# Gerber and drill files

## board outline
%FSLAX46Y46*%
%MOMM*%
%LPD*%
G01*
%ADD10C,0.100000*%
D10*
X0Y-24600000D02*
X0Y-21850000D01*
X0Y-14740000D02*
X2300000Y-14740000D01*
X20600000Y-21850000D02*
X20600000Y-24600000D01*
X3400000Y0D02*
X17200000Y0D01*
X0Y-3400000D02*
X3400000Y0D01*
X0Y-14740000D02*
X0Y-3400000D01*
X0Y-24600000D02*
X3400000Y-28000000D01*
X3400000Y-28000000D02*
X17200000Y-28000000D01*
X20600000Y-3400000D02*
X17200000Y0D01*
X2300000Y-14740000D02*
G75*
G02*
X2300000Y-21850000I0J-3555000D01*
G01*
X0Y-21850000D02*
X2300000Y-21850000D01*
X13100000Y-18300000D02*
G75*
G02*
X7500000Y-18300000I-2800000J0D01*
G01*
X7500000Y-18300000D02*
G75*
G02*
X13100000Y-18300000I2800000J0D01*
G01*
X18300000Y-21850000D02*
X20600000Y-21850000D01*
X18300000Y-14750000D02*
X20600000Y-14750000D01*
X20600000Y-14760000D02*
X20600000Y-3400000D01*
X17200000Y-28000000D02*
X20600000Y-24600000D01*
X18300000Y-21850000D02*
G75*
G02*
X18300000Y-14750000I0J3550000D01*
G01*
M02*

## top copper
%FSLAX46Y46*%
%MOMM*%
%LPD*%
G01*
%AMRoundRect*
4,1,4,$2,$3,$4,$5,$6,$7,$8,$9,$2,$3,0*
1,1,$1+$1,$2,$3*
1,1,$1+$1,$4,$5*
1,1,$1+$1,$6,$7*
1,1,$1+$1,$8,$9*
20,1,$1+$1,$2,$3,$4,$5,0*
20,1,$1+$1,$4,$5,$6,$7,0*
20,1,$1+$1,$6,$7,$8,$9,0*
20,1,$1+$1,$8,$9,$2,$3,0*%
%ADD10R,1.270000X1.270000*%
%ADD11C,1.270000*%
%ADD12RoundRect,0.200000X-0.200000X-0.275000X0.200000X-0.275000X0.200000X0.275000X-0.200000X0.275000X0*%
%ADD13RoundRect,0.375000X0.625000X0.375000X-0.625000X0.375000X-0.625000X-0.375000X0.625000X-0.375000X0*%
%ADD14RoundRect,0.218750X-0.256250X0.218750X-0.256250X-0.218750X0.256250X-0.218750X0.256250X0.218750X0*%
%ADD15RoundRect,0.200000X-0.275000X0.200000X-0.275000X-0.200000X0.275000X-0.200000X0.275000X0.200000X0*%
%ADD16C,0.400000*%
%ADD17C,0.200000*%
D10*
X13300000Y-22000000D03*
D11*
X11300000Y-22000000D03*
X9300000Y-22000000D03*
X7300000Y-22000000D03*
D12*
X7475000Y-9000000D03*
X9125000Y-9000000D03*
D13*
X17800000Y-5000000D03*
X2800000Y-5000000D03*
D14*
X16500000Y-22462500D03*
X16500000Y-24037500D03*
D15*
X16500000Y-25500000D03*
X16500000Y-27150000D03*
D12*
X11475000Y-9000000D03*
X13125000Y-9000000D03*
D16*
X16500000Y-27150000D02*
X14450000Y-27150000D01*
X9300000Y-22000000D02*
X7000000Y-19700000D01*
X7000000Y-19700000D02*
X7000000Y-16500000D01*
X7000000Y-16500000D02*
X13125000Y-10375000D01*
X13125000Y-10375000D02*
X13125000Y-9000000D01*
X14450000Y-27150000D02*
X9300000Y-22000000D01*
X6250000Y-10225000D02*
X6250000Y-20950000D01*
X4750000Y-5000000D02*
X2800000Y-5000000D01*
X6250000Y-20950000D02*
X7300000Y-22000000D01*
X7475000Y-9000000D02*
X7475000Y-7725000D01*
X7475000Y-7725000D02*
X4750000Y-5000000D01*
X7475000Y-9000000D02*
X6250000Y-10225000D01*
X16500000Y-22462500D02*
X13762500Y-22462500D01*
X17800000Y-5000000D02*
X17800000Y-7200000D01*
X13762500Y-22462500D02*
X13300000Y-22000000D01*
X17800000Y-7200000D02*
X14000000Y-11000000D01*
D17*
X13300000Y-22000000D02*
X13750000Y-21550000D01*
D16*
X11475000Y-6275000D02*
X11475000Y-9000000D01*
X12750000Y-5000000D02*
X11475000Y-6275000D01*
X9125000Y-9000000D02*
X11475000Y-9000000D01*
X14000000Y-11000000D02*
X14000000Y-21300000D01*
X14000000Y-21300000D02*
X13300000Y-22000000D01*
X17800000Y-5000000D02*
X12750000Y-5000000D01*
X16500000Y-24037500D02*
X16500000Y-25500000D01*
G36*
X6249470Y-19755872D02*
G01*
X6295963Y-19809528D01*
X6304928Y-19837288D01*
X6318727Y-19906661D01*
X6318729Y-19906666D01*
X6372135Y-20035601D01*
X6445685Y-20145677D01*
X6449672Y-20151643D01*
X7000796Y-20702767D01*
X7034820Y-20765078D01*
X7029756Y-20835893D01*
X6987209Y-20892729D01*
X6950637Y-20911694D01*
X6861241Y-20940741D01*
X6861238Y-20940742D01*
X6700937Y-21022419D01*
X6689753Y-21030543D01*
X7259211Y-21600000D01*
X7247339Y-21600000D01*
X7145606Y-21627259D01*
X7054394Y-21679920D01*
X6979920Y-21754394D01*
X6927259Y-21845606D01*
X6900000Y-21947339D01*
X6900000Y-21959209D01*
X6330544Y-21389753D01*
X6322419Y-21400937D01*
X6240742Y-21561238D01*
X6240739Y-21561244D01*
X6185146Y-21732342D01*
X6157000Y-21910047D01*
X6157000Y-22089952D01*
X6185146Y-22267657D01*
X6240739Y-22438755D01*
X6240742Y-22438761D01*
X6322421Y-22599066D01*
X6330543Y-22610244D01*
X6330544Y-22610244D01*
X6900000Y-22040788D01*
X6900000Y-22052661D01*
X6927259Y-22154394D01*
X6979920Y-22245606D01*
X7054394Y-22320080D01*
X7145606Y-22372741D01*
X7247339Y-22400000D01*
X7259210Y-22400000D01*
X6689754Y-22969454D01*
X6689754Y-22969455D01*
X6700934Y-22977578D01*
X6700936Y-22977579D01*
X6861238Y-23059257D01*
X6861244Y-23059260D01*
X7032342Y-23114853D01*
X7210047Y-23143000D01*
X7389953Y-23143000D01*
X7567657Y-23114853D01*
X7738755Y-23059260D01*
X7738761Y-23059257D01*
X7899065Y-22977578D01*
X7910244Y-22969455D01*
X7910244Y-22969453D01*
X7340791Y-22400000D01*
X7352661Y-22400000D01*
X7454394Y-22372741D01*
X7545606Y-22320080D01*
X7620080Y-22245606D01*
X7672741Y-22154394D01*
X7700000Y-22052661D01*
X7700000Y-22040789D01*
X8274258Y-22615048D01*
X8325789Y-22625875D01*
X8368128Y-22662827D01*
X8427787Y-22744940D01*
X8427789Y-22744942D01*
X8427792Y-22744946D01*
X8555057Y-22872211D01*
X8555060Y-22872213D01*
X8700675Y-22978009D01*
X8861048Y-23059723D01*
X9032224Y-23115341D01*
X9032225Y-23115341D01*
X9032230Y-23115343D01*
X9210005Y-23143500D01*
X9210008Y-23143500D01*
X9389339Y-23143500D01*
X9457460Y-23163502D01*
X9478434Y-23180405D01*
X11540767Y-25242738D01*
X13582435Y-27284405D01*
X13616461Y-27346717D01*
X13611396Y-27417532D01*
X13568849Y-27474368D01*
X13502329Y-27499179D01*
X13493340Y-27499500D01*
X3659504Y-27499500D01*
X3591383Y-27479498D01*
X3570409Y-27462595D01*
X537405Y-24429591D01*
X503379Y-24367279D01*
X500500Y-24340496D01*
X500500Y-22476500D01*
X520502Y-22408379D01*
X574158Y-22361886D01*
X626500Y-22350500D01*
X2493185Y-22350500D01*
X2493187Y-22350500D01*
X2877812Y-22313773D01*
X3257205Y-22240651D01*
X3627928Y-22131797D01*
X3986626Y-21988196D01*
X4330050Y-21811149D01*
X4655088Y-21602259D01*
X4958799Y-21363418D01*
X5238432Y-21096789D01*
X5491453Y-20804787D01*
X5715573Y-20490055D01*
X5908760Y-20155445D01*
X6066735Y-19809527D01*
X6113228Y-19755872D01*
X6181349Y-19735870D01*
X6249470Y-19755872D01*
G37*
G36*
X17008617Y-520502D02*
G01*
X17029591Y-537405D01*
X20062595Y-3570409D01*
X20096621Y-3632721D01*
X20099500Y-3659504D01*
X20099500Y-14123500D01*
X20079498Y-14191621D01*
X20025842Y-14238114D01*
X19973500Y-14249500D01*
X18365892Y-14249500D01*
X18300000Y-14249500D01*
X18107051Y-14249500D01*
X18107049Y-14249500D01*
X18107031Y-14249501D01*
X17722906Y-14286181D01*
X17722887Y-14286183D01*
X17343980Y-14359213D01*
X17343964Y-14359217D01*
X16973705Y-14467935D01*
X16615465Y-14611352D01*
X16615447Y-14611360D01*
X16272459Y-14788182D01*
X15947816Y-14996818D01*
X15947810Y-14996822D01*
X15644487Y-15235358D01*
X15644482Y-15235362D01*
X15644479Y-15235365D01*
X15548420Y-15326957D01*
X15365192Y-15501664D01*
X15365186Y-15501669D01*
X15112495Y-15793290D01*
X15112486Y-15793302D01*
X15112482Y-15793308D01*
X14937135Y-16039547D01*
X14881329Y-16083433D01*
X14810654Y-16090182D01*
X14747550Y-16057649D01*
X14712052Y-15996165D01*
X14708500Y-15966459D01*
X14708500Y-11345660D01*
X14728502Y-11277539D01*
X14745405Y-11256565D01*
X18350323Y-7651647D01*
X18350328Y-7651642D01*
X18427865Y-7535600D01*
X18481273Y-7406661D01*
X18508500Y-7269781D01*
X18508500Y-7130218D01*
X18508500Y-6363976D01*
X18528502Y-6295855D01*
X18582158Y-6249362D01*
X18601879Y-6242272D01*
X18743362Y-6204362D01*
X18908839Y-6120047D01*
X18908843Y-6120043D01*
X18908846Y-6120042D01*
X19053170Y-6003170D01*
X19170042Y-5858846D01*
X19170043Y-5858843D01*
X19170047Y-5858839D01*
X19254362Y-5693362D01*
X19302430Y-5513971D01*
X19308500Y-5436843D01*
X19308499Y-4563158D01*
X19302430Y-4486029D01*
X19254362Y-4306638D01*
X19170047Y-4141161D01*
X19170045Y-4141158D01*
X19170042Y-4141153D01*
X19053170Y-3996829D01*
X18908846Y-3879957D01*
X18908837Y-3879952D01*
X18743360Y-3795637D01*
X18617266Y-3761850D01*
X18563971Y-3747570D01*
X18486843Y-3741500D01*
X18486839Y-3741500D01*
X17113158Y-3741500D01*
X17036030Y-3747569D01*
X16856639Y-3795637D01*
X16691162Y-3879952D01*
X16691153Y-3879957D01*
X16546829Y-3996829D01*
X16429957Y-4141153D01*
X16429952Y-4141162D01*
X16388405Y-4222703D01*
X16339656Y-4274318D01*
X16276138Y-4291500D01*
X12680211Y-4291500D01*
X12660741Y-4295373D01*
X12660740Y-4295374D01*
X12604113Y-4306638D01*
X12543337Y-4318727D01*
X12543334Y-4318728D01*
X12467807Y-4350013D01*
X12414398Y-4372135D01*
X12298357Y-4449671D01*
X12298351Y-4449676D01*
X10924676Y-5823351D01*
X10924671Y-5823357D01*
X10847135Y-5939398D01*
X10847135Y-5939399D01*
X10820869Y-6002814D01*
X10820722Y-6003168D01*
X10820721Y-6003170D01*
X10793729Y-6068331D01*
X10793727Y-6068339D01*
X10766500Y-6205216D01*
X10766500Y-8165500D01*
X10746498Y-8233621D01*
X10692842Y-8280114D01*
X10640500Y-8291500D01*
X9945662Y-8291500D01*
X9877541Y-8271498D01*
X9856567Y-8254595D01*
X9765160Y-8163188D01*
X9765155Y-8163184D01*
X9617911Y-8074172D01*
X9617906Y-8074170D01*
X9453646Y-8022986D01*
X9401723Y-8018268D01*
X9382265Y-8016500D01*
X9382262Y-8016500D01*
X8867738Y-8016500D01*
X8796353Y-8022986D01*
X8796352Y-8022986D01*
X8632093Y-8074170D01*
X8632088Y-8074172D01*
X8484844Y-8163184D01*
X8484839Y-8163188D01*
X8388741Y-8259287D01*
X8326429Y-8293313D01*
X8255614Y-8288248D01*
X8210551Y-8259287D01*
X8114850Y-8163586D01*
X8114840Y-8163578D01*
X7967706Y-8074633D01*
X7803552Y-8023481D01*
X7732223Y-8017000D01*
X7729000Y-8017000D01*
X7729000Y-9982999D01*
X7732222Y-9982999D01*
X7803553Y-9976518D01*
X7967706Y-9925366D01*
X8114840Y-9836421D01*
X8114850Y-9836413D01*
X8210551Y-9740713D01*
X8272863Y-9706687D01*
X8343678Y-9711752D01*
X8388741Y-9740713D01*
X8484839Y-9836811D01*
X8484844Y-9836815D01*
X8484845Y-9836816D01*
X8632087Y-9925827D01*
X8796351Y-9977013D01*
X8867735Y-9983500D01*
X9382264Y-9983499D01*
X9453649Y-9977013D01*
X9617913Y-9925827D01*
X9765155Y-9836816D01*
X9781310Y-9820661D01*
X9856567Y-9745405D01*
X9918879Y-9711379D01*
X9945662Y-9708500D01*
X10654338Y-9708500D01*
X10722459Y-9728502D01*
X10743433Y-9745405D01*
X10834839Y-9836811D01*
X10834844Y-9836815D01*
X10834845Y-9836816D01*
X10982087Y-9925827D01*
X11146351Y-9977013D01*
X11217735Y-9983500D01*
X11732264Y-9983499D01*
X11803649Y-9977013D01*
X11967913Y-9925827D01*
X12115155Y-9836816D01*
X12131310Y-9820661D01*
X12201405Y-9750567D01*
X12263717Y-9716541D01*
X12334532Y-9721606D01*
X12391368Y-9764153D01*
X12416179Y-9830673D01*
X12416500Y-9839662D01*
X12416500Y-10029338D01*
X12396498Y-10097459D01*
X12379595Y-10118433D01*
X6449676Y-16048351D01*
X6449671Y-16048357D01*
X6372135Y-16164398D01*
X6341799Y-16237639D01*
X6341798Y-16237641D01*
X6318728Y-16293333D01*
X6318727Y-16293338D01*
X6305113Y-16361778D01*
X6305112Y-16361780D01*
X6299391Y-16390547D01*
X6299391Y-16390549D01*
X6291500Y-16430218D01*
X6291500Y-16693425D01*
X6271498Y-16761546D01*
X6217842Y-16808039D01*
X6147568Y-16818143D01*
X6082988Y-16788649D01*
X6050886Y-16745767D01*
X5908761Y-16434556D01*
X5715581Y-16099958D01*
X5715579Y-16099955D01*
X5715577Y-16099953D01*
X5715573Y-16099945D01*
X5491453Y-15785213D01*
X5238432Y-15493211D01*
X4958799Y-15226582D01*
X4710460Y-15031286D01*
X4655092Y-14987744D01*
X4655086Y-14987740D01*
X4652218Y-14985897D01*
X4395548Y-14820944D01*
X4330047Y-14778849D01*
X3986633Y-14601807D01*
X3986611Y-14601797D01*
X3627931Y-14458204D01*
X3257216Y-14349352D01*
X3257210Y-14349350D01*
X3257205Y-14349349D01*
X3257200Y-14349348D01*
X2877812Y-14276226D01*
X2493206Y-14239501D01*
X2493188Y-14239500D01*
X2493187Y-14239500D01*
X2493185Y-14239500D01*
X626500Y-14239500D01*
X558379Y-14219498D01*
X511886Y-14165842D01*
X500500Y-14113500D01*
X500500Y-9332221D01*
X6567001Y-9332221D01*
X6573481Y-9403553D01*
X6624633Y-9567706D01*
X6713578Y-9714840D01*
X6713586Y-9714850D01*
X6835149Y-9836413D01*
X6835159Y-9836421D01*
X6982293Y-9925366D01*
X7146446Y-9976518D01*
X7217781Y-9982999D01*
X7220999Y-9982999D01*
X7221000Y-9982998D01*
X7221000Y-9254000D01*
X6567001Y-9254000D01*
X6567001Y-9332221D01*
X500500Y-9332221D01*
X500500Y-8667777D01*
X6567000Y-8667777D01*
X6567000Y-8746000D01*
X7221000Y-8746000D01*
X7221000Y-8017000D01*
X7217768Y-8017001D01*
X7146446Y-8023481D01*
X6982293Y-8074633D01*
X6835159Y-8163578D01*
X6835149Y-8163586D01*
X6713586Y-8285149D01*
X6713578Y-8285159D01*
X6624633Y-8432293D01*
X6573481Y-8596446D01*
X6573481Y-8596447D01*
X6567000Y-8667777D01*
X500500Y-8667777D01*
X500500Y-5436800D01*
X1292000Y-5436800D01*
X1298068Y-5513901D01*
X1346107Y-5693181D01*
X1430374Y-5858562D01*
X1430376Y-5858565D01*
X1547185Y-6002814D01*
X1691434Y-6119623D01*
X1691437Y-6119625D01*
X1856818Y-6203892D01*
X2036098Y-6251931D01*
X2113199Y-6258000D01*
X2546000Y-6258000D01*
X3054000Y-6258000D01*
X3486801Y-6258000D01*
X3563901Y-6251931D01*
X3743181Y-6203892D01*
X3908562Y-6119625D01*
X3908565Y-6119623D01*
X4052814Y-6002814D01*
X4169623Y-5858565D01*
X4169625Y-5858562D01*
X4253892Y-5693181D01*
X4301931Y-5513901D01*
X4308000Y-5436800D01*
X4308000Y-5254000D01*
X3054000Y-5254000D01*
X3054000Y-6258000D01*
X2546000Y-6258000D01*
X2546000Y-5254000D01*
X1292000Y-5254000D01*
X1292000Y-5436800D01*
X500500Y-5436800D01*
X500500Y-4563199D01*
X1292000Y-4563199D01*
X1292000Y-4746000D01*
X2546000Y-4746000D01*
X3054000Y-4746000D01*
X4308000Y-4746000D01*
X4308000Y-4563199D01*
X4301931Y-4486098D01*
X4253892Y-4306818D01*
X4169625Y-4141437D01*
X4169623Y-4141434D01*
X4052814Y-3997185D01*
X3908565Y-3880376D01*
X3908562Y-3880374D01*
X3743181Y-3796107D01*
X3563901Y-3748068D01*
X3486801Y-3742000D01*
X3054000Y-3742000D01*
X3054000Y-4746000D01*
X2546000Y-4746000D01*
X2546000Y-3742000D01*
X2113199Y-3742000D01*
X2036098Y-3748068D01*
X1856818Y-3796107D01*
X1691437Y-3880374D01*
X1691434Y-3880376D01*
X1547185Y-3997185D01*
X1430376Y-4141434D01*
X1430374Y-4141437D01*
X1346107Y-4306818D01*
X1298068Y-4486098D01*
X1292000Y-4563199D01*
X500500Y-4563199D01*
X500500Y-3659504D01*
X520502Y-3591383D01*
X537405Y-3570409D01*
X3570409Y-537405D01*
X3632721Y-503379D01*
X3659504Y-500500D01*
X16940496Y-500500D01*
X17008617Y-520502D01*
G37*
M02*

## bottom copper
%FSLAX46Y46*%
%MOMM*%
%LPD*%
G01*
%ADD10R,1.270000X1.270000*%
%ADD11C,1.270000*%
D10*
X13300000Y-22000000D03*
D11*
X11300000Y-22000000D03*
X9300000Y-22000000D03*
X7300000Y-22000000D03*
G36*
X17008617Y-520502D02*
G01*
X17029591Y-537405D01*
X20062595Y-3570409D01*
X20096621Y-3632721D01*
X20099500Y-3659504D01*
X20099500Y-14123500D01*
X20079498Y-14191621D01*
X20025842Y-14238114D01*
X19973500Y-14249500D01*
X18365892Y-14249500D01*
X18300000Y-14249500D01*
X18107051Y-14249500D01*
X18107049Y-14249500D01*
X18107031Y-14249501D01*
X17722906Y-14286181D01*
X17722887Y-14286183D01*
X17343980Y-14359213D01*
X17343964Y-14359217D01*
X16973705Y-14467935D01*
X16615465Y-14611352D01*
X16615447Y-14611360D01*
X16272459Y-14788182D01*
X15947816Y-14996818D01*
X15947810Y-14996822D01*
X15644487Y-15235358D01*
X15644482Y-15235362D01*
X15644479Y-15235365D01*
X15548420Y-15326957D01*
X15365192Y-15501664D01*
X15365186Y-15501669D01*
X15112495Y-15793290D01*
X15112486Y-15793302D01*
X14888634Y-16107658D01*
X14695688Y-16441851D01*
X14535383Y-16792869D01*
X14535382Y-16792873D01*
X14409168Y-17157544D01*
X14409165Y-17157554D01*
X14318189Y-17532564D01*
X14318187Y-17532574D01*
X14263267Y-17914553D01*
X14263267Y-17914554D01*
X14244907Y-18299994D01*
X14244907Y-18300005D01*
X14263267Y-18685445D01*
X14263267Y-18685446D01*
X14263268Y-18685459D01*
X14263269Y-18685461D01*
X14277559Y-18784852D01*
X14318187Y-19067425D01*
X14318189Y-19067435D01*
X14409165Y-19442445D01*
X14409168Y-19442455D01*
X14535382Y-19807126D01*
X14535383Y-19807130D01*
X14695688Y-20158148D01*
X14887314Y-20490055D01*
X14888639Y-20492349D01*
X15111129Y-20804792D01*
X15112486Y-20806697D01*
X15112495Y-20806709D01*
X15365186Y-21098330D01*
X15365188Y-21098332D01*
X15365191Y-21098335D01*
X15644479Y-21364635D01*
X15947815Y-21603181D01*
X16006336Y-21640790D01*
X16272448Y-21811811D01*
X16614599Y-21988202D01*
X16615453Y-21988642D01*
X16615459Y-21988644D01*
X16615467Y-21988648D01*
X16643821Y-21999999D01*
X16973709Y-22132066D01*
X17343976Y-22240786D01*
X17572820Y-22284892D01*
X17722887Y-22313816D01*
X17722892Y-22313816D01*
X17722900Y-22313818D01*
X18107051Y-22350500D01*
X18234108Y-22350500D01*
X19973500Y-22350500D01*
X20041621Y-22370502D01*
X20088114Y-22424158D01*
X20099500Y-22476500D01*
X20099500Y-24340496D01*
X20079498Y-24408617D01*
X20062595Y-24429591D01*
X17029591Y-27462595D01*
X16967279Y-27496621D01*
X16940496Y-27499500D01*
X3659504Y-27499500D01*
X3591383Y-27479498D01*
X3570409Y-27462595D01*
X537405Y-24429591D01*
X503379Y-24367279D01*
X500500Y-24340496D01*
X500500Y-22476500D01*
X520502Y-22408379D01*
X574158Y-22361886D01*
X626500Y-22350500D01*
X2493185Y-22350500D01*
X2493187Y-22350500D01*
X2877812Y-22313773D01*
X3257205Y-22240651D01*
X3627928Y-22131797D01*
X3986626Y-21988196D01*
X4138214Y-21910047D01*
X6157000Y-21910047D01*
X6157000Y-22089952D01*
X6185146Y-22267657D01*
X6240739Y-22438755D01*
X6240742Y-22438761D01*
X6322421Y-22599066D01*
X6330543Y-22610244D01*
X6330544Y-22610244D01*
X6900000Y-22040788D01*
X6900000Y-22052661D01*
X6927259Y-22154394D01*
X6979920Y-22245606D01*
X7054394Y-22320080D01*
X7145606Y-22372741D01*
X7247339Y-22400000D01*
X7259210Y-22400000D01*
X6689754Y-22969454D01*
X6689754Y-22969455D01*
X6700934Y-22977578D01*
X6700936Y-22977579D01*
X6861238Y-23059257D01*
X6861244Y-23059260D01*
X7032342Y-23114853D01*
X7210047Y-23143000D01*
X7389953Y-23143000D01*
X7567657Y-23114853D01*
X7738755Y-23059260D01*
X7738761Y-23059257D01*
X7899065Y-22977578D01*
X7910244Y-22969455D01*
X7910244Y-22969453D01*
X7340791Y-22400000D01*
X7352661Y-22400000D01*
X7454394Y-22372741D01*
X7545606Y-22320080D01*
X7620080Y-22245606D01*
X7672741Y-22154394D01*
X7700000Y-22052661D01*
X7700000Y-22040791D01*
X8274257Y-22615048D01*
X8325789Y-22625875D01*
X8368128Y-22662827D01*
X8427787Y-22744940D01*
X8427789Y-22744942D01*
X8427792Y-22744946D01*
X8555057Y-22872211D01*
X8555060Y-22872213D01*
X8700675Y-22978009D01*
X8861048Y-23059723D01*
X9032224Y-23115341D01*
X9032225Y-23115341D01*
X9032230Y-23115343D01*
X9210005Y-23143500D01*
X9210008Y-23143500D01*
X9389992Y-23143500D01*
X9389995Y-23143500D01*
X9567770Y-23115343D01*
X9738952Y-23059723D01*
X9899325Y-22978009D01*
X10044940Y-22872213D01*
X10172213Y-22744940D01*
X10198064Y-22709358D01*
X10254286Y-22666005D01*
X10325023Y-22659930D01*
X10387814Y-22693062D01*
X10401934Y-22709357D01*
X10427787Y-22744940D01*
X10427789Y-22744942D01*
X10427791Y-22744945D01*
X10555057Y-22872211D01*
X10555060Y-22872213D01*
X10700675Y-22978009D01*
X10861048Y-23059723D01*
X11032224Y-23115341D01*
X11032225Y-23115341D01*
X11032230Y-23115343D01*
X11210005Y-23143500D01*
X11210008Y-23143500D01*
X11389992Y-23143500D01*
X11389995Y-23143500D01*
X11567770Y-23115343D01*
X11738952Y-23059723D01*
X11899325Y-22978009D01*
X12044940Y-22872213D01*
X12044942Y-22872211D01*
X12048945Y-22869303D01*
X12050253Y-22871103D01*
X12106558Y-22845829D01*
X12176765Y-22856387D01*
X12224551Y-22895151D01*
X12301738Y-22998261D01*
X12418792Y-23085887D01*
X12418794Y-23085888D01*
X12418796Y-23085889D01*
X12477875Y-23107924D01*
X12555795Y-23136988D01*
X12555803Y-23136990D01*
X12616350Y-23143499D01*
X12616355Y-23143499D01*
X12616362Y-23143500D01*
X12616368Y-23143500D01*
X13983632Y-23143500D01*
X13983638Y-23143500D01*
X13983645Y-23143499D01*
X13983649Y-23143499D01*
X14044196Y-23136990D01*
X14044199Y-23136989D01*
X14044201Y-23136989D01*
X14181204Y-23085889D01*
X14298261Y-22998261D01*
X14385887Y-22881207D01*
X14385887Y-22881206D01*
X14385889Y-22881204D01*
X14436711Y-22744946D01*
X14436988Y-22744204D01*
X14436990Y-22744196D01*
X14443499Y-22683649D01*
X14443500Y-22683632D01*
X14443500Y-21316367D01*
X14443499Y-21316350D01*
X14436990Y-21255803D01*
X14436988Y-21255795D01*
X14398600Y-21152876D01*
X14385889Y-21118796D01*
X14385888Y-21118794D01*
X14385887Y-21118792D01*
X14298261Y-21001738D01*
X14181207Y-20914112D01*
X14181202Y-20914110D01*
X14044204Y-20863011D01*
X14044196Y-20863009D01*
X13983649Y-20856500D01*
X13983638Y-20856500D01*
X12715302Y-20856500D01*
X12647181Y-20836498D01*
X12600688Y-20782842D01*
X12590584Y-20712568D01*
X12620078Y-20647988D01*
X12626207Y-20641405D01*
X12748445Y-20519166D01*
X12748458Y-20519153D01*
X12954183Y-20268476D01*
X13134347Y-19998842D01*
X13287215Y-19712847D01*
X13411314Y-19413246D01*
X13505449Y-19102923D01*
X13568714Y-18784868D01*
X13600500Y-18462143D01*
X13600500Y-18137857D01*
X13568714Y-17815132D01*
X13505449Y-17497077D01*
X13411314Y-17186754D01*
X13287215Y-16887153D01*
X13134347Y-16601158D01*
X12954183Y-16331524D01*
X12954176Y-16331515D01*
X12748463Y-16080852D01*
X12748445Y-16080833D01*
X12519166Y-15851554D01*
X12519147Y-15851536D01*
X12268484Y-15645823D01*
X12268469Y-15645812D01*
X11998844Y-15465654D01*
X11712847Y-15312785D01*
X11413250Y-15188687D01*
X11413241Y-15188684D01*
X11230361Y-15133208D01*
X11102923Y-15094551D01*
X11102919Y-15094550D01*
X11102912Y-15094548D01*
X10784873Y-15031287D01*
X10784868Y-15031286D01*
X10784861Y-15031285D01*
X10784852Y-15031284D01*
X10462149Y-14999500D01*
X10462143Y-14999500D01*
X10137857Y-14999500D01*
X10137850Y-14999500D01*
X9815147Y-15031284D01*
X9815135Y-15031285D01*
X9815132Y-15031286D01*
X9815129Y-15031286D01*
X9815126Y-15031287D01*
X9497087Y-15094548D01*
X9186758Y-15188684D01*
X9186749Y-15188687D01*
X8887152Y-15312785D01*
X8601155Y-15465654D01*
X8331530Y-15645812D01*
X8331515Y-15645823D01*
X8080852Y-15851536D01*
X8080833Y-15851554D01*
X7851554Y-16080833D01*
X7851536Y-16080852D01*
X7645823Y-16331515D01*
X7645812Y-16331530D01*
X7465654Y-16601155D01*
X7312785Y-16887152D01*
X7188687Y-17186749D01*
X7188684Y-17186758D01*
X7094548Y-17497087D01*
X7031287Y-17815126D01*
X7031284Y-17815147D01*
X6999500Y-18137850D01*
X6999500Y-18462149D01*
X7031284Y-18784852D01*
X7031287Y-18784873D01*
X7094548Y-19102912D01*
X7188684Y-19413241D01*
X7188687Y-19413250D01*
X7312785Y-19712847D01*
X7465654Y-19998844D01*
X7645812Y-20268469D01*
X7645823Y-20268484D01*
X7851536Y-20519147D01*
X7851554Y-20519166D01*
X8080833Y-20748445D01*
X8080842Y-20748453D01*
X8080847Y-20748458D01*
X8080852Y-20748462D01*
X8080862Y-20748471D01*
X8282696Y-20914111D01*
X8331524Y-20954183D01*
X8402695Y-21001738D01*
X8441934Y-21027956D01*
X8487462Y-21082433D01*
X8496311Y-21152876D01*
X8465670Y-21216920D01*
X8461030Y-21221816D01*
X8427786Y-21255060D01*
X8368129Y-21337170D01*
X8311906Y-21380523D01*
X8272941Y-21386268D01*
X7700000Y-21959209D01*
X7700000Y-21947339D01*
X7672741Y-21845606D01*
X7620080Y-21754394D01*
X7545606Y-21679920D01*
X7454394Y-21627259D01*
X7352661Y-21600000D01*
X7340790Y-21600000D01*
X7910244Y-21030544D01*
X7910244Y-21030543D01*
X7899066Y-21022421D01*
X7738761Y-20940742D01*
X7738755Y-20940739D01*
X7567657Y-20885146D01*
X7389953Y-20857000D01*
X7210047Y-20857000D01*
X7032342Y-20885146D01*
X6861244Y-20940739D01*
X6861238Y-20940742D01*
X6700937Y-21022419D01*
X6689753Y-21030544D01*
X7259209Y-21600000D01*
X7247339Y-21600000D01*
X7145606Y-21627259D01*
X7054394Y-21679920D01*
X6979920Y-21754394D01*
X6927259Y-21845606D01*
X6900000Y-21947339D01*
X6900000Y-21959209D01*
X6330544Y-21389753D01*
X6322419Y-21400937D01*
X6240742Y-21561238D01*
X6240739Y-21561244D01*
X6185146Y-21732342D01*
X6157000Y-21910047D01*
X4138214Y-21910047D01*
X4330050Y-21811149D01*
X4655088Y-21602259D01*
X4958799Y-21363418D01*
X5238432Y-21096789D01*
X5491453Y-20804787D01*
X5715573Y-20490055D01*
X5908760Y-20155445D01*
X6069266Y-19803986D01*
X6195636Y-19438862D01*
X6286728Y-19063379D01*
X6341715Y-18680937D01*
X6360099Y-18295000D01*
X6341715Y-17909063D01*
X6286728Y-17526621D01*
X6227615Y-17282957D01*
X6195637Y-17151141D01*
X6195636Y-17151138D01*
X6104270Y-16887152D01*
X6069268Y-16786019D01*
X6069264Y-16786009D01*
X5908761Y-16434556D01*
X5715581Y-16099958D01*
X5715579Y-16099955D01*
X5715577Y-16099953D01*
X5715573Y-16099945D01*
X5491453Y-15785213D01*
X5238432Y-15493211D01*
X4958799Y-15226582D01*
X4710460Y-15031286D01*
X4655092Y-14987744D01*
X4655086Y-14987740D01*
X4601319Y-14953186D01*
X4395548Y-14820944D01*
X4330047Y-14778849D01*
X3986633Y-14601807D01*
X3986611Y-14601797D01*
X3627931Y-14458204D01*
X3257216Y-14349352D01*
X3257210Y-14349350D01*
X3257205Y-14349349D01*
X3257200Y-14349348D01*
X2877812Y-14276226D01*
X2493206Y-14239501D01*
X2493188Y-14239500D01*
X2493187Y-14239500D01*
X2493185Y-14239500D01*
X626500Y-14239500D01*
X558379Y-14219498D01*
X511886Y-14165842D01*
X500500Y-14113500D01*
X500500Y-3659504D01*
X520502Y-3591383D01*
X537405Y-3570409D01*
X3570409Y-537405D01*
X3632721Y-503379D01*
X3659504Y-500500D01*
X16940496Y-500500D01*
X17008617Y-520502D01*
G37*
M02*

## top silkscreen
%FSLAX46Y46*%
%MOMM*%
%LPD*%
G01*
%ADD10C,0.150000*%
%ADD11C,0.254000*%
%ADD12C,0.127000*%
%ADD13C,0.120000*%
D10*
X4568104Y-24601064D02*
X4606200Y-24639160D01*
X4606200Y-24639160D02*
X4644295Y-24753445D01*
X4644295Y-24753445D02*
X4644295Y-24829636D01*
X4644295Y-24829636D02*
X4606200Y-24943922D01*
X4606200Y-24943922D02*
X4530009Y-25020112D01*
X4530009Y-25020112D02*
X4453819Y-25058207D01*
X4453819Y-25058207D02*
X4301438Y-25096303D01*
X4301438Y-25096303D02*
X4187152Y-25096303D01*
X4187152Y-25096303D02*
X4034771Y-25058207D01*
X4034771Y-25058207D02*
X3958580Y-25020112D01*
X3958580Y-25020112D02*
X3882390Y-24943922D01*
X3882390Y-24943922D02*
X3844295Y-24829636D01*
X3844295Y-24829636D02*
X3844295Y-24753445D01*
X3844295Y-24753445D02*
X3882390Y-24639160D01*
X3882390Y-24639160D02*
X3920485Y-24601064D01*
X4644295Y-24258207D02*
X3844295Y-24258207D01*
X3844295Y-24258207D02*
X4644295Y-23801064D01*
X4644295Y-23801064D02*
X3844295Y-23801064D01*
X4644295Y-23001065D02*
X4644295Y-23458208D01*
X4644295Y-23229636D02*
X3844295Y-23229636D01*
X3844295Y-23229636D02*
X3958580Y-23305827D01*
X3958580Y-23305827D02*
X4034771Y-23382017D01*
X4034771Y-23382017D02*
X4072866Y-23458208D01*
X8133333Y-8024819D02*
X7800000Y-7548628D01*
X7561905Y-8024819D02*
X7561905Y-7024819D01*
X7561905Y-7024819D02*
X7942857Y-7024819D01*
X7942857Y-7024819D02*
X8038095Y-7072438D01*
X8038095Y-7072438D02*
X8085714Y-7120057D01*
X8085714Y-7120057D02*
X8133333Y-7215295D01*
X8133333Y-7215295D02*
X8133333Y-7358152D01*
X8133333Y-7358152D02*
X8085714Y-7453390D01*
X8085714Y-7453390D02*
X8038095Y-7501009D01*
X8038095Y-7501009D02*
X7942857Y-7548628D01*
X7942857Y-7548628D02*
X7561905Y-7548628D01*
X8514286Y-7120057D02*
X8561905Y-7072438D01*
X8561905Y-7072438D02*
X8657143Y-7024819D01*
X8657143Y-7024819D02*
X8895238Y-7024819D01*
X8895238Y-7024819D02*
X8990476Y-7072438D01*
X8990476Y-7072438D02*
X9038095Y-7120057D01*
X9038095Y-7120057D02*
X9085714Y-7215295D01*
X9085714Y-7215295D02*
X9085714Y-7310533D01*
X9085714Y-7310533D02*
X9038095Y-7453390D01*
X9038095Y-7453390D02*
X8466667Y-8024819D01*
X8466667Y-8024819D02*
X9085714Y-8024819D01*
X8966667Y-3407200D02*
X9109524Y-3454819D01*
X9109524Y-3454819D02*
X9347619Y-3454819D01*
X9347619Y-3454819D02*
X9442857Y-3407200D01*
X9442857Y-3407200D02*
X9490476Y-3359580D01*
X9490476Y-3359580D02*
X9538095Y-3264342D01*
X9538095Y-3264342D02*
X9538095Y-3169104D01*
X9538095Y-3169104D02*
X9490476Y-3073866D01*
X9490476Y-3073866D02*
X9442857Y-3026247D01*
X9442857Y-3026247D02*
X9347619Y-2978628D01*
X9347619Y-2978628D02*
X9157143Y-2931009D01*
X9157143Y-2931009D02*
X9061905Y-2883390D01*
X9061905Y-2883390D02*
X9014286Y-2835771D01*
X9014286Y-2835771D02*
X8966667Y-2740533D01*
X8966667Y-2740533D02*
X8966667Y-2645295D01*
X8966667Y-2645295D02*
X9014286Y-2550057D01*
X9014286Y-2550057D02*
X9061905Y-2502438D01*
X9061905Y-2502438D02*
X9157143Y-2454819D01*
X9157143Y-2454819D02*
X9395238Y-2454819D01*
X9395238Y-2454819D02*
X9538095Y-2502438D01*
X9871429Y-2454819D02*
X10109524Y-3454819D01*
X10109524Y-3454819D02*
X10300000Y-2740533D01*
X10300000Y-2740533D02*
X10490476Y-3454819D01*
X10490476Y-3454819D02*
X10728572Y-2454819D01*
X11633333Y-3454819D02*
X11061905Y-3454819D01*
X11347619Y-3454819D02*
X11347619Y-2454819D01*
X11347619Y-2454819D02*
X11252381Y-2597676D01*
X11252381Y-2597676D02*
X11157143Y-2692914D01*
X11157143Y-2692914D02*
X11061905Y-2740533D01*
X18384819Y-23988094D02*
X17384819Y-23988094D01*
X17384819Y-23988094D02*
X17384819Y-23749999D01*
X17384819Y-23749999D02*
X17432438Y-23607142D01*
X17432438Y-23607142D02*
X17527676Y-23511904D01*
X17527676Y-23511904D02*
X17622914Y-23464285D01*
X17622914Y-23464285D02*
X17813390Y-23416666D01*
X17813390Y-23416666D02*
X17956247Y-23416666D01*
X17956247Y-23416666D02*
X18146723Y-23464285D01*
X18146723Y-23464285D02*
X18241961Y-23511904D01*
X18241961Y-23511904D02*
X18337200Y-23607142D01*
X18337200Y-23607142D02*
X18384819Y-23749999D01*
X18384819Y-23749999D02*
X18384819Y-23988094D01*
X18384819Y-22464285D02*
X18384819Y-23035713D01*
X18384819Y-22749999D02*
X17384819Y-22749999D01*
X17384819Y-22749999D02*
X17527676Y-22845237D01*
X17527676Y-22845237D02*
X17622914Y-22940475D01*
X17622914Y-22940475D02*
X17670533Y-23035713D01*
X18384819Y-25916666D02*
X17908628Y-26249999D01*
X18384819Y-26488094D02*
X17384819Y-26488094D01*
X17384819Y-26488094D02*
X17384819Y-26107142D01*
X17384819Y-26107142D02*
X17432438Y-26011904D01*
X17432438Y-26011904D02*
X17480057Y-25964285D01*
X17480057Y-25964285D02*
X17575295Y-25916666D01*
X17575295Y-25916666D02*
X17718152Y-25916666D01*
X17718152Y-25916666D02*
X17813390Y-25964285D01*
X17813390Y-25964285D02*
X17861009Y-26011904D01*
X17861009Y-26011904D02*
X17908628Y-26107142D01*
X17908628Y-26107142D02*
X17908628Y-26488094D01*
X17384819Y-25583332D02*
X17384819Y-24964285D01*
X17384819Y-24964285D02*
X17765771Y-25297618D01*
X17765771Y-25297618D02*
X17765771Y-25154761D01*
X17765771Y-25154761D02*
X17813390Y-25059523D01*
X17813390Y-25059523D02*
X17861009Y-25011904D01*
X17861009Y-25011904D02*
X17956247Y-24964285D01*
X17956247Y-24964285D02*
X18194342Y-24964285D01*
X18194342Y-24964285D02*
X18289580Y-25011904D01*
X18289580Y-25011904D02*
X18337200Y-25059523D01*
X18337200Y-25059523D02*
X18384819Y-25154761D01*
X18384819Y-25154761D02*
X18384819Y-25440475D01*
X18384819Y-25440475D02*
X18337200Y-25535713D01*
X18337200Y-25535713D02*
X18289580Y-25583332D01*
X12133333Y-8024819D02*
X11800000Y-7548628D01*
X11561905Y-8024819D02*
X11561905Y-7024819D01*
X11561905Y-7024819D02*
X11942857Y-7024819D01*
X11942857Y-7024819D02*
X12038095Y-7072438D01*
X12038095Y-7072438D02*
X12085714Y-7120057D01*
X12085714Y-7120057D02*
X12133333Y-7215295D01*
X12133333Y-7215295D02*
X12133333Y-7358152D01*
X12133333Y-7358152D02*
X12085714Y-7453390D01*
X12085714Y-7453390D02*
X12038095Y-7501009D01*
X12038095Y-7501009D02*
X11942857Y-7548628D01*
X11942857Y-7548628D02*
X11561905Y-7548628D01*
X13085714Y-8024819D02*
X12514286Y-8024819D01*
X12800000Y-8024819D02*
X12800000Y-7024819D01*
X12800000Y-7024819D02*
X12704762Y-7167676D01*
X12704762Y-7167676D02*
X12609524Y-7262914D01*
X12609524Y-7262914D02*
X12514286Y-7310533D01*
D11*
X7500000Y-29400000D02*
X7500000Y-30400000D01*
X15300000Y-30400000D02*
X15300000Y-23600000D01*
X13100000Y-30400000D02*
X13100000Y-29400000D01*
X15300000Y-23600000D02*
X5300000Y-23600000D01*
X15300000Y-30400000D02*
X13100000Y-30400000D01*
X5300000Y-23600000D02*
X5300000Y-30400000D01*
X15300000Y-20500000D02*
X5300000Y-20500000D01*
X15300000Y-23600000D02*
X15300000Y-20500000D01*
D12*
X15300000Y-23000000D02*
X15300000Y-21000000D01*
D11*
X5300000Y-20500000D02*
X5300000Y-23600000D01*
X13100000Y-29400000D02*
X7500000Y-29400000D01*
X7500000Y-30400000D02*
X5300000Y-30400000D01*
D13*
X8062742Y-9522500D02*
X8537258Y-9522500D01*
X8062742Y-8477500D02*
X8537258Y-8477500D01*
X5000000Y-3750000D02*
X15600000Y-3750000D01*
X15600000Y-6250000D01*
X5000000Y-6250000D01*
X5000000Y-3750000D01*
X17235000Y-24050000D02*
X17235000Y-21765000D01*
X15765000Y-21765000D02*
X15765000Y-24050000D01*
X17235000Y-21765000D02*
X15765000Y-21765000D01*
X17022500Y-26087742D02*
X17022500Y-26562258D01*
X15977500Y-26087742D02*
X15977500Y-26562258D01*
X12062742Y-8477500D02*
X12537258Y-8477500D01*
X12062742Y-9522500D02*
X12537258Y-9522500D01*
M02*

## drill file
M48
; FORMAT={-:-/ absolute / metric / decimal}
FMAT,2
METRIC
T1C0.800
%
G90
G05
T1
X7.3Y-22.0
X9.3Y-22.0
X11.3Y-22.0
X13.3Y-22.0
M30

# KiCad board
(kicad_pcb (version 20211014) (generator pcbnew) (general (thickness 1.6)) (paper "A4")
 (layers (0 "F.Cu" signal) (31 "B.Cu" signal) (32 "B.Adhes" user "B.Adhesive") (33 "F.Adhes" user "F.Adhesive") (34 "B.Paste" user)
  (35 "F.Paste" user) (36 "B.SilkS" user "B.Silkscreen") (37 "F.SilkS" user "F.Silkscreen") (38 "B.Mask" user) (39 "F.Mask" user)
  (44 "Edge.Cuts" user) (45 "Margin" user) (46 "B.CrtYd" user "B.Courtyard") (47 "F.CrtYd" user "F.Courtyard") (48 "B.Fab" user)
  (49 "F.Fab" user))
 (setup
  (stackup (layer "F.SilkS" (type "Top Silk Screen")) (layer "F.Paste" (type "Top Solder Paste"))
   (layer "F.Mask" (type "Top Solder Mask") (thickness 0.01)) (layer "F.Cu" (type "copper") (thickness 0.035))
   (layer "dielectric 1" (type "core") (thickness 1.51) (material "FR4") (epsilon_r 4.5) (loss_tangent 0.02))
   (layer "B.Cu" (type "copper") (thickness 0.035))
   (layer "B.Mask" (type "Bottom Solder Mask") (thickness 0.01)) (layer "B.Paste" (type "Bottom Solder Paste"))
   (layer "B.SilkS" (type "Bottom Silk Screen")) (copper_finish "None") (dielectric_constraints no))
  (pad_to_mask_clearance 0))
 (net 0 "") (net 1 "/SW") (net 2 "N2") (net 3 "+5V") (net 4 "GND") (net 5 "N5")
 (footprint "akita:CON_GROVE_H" (layer "F.Cu") (at 10.3 22 180)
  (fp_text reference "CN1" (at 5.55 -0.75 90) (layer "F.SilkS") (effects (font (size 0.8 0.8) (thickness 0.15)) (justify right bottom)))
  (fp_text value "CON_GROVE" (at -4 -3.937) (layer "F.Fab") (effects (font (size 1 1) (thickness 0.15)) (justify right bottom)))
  (fp_line (start 2.8 -7.4) (end 2.8 -8.4) (layer "F.SilkS") (width 0.254))
  (fp_line (start -5 -8.4) (end -5 -1.6) (layer "F.SilkS") (width 0.254))
  (fp_line (start -2.8 -8.4) (end -2.8 -7.4) (layer "F.SilkS") (width 0.254))
  (fp_line (start -5 -1.6) (end 5 -1.6) (layer "F.SilkS") (width 0.254))
  (fp_line (start -5 -8.4) (end -2.8 -8.4) (layer "F.SilkS") (width 0.254))
  (fp_line (start 5 -1.6) (end 5 -8.4) (layer "F.SilkS") (width 0.254))
  (fp_line (start -5 1.5) (end 5 1.5) (layer "F.SilkS") (width 0.254))
  (fp_line (start -5 -1.6) (end -5 1.5) (layer "F.SilkS") (width 0.254))
  (fp_line (start -5 -1) (end -5 1) (layer "F.SilkS") (width 0.127))
  (fp_line (start 5 1.5) (end 5 -1.6) (layer "F.SilkS") (width 0.254))
  (fp_line (start -2.8 -7.4) (end 2.8 -7.4) (layer "F.SilkS") (width 0.254))
  (fp_line (start 2.8 -8.4) (end 5 -8.4) (layer "F.SilkS") (width 0.254))
  (pad "1" thru_hole rect locked (at -3 0 180) (size 1.27 1.27) (drill 0.8) (layers *.Cu *.Mask) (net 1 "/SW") (solder_mask_margin 0.1016))
  (pad "2" thru_hole circle locked (at -1 0 180) (size 1.27 1.27) (drill 0.8) (layers *.Cu *.Mask) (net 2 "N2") (solder_mask_margin 0.1016))
  (pad "3" thru_hole circle locked (at 1 0 180) (size 1.27 1.27) (drill 0.8) (layers *.Cu *.Mask) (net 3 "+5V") (solder_mask_margin 0.1016))
  (pad "4" thru_hole circle locked (at 3 0 180) (size 1.27 1.27) (drill 0.8) (layers *.Cu *.Mask) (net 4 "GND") (solder_mask_margin 0.1016)))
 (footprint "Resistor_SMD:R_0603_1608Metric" (layer "F.Cu") (at 8.3 9)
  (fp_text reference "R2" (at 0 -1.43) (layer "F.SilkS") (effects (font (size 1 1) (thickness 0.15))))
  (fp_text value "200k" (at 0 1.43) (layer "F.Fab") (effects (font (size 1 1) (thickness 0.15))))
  (fp_line (start -0.237258 0.5225) (end 0.237258 0.5225) (layer "F.SilkS") (width 0.12))
  (fp_line (start -0.237258 -0.5225) (end 0.237258 -0.5225) (layer "F.SilkS") (width 0.12))
  (pad "1" smd roundrect locked (at -0.825 0) (size 0.8 0.95) (layers "F.Cu" "F.Paste" "F.Mask") (roundrect_rratio 0.25) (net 4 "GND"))
  (pad "2" smd roundrect locked (at 0.825 0) (size 0.8 0.95) (layers "F.Cu" "F.Paste" "F.Mask") (roundrect_rratio 0.25) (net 1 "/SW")))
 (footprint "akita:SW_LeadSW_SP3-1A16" (layer "F.Cu") (at 10.3 5 180)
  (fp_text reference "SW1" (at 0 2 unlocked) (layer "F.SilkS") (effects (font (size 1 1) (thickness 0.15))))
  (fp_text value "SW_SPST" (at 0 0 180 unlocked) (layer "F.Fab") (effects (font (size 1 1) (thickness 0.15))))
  (fp_rect (start -5.3 -1.25) (end 5.3 1.25) (layer "F.SilkS") (width 0.12) (fill none))
  (pad "1" smd roundrect (at -7.5 0 180) (size 2 1.5) (layers "F.Cu" "F.Paste" "F.Mask") (roundrect_rratio 0.25) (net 1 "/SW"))
  (pad "2" smd roundrect (at 7.5 0 180) (size 2 1.5) (layers "F.Cu" "F.Paste" "F.Mask") (roundrect_rratio 0.25) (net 4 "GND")))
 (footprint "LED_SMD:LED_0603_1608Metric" (layer "F.Cu") (at 16.5 23.25 -90)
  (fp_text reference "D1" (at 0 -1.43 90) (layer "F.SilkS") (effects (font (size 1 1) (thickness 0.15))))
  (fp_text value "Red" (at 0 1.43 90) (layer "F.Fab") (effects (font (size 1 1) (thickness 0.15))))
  (fp_line (start 0.8 -0.735) (end -1.485 -0.735) (layer "F.SilkS") (width 0.12))
  (fp_line (start -1.485 0.735) (end 0.8 0.735) (layer "F.SilkS") (width 0.12))
  (fp_line (start -1.485 -0.735) (end -1.485 0.735) (layer "F.SilkS") (width 0.12))
  (pad "1" smd roundrect locked (at -0.7875 0 270) (size 0.875 0.95) (layers "F.Cu" "F.Paste" "F.Mask") (roundrect_rratio 0.25)
   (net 1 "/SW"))
  (pad "2" smd roundrect locked (at 0.7875 0 270) (size 0.875 0.95) (layers "F.Cu" "F.Paste" "F.Mask") (roundrect_rratio 0.25) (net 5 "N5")))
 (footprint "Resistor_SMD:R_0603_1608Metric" (layer "F.Cu") (at 16.5 26.325 -90)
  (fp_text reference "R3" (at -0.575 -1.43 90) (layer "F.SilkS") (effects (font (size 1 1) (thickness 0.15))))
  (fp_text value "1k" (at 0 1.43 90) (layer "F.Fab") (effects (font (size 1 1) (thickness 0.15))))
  (fp_line (start -0.237258 -0.5225) (end 0.237258 -0.5225) (layer "F.SilkS") (width 0.12))
  (fp_line (start -0.237258 0.5225) (end 0.237258 0.5225) (layer "F.SilkS") (width 0.12))
  (pad "1" smd roundrect locked (at -0.825 0 270) (size 0.8 0.95) (layers "F.Cu" "F.Paste" "F.Mask") (roundrect_rratio 0.25) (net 5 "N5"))
  (pad "2" smd roundrect locked (at 0.825 0 270) (size 0.8 0.95) (layers "F.Cu" "F.Paste" "F.Mask") (roundrect_rratio 0.25) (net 3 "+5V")))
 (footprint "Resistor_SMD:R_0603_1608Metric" (layer "F.Cu") (at 12.3 9)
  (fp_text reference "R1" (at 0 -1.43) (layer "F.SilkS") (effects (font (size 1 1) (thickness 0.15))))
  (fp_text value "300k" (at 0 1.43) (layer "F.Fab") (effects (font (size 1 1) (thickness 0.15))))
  (fp_line (start -0.237258 -0.5225) (end 0.237258 -0.5225) (layer "F.SilkS") (width 0.12))
  (fp_line (start -0.237258 0.5225) (end 0.237258 0.5225) (layer "F.SilkS") (width 0.12))
  (pad "1" smd roundrect locked (at -0.825 0) (size 0.8 0.95) (layers "F.Cu" "F.Paste" "F.Mask") (roundrect_rratio 0.25) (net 1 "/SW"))
  (pad "2" smd roundrect locked (at 0.825 0) (size 0.8 0.95) (layers "F.Cu" "F.Paste" "F.Mask") (roundrect_rratio 0.25) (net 3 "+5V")))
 (gr_line (start 0 24.6) (end 0 21.85) (layer "Edge.Cuts") (width 0.1))
 (gr_line (start 0 14.74) (end 2.3 14.74) (layer "Edge.Cuts") (width 0.1))
 (gr_line (start 20.6 21.85) (end 20.6 24.6) (layer "Edge.Cuts") (width 0.1))
 (gr_line (start 3.4 0) (end 17.2 0) (layer "Edge.Cuts") (width 0.1))
 (gr_line (start 0 3.4) (end 3.4 0) (layer "Edge.Cuts") (width 0.1))
 (gr_line (start 0 14.74) (end 0 3.4) (layer "Edge.Cuts") (width 0.1))
 (gr_line (start 0 24.6) (end 3.4 28) (layer "Edge.Cuts") (width 0.1))
 (gr_line (start 3.4 28) (end 17.2 28) (layer "Edge.Cuts") (width 0.1))
 (gr_line (start 20.6 3.4) (end 17.2 0) (layer "Edge.Cuts") (width 0.1))
 (gr_arc (start 2.3 14.74) (mid 5.855 18.295) (end 2.3 21.85) (layer "Edge.Cuts") (width 0.1))
 (gr_line (start 0 21.85) (end 2.3 21.85) (layer "Edge.Cuts") (width 0.1))
 (gr_circle (center 10.3 18.3) (end 13.1 18.3) (layer "Edge.Cuts") (width 0.1) (fill none))
 (gr_line (start 18.3 21.85) (end 20.6 21.85) (layer "Edge.Cuts") (width 0.1))
 (gr_line (start 18.3 14.75) (end 20.6 14.75) (layer "Edge.Cuts") (width 0.1))
 (gr_line (start 20.6 14.76) (end 20.6 3.4) (layer "Edge.Cuts") (width 0.1))
 (gr_line (start 17.2 28) (end 20.6 24.6) (layer "Edge.Cuts") (width 0.1))
 (gr_arc (start 18.3 21.85) (mid 14.75 18.3) (end 18.3 14.75) (layer "Edge.Cuts") (width 0.1))
 (segment (start 16.5 27.15) (end 14.45 27.15) (width 0.4) (layer "F.Cu") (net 3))
 (segment (start 9.3 22) (end 7 19.7) (width 0.4) (layer "F.Cu") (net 3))
 (segment (start 7 19.7) (end 7 16.5) (width 0.4) (layer "F.Cu") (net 3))
 (segment (start 7 16.5) (end 13.125 10.375) (width 0.4) (layer "F.Cu") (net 3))
 (segment (start 13.125 10.375) (end 13.125 9) (width 0.4) (layer "F.Cu") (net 3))
 (segment (start 14.45 27.15) (end 9.3 22) (width 0.4) (layer "F.Cu") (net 3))
 (segment (start 6.25 10.225) (end 6.25 20.95) (width 0.4) (layer "F.Cu") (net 4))
 (segment (start 4.75 5) (end 2.8 5) (width 0.4) (layer "F.Cu") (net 4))
 (segment (start 6.25 20.95) (end 7.3 22) (width 0.4) (layer "F.Cu") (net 4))
 (segment (start 7.475 9) (end 7.475 7.725) (width 0.4) (layer "F.Cu") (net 4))
 (segment (start 7.475 7.725) (end 4.75 5) (width 0.4) (layer "F.Cu") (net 4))
 (segment (start 7.475 9) (end 6.25 10.225) (width 0.4) (layer "F.Cu") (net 4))
 (segment (start 16.5 22.4625) (end 13.7625 22.4625) (width 0.4) (layer "F.Cu") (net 1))
 (segment (start 17.8 5) (end 17.8 7.2) (width 0.4) (layer "F.Cu") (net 1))
 (segment (start 13.7625 22.4625) (end 13.3 22) (width 0.4) (layer "F.Cu") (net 1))
 (segment (start 17.8 7.2) (end 14 11) (width 0.4) (layer "F.Cu") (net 1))
 (segment (start 13.3 22) (end 13.75 21.55) (width 0.2) (layer "F.Cu") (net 1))
 (segment (start 11.475 6.275) (end 11.475 9) (width 0.4) (layer "F.Cu") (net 1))
 (segment (start 12.75 5) (end 11.475 6.275) (width 0.4) (layer "F.Cu") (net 1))
 (segment (start 9.125 9) (end 11.475 9) (width 0.4) (layer "F.Cu") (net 1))
 (segment (start 14 11) (end 14 21.3) (width 0.4) (layer "F.Cu") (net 1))
 (segment (start 14 21.3) (end 13.3 22) (width 0.4) (layer "F.Cu") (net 1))
 (segment (start 17.8 5) (end 12.75 5) (width 0.4) (layer "F.Cu") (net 1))
 (segment (start 16.5 24.0375) (end 16.5 25.5) (width 0.4) (layer "F.Cu") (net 5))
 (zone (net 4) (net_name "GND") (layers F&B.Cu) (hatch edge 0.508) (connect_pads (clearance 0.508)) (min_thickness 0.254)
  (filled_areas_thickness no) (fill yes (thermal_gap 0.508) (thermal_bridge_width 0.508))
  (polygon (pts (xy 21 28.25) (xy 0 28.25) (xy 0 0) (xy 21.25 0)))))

